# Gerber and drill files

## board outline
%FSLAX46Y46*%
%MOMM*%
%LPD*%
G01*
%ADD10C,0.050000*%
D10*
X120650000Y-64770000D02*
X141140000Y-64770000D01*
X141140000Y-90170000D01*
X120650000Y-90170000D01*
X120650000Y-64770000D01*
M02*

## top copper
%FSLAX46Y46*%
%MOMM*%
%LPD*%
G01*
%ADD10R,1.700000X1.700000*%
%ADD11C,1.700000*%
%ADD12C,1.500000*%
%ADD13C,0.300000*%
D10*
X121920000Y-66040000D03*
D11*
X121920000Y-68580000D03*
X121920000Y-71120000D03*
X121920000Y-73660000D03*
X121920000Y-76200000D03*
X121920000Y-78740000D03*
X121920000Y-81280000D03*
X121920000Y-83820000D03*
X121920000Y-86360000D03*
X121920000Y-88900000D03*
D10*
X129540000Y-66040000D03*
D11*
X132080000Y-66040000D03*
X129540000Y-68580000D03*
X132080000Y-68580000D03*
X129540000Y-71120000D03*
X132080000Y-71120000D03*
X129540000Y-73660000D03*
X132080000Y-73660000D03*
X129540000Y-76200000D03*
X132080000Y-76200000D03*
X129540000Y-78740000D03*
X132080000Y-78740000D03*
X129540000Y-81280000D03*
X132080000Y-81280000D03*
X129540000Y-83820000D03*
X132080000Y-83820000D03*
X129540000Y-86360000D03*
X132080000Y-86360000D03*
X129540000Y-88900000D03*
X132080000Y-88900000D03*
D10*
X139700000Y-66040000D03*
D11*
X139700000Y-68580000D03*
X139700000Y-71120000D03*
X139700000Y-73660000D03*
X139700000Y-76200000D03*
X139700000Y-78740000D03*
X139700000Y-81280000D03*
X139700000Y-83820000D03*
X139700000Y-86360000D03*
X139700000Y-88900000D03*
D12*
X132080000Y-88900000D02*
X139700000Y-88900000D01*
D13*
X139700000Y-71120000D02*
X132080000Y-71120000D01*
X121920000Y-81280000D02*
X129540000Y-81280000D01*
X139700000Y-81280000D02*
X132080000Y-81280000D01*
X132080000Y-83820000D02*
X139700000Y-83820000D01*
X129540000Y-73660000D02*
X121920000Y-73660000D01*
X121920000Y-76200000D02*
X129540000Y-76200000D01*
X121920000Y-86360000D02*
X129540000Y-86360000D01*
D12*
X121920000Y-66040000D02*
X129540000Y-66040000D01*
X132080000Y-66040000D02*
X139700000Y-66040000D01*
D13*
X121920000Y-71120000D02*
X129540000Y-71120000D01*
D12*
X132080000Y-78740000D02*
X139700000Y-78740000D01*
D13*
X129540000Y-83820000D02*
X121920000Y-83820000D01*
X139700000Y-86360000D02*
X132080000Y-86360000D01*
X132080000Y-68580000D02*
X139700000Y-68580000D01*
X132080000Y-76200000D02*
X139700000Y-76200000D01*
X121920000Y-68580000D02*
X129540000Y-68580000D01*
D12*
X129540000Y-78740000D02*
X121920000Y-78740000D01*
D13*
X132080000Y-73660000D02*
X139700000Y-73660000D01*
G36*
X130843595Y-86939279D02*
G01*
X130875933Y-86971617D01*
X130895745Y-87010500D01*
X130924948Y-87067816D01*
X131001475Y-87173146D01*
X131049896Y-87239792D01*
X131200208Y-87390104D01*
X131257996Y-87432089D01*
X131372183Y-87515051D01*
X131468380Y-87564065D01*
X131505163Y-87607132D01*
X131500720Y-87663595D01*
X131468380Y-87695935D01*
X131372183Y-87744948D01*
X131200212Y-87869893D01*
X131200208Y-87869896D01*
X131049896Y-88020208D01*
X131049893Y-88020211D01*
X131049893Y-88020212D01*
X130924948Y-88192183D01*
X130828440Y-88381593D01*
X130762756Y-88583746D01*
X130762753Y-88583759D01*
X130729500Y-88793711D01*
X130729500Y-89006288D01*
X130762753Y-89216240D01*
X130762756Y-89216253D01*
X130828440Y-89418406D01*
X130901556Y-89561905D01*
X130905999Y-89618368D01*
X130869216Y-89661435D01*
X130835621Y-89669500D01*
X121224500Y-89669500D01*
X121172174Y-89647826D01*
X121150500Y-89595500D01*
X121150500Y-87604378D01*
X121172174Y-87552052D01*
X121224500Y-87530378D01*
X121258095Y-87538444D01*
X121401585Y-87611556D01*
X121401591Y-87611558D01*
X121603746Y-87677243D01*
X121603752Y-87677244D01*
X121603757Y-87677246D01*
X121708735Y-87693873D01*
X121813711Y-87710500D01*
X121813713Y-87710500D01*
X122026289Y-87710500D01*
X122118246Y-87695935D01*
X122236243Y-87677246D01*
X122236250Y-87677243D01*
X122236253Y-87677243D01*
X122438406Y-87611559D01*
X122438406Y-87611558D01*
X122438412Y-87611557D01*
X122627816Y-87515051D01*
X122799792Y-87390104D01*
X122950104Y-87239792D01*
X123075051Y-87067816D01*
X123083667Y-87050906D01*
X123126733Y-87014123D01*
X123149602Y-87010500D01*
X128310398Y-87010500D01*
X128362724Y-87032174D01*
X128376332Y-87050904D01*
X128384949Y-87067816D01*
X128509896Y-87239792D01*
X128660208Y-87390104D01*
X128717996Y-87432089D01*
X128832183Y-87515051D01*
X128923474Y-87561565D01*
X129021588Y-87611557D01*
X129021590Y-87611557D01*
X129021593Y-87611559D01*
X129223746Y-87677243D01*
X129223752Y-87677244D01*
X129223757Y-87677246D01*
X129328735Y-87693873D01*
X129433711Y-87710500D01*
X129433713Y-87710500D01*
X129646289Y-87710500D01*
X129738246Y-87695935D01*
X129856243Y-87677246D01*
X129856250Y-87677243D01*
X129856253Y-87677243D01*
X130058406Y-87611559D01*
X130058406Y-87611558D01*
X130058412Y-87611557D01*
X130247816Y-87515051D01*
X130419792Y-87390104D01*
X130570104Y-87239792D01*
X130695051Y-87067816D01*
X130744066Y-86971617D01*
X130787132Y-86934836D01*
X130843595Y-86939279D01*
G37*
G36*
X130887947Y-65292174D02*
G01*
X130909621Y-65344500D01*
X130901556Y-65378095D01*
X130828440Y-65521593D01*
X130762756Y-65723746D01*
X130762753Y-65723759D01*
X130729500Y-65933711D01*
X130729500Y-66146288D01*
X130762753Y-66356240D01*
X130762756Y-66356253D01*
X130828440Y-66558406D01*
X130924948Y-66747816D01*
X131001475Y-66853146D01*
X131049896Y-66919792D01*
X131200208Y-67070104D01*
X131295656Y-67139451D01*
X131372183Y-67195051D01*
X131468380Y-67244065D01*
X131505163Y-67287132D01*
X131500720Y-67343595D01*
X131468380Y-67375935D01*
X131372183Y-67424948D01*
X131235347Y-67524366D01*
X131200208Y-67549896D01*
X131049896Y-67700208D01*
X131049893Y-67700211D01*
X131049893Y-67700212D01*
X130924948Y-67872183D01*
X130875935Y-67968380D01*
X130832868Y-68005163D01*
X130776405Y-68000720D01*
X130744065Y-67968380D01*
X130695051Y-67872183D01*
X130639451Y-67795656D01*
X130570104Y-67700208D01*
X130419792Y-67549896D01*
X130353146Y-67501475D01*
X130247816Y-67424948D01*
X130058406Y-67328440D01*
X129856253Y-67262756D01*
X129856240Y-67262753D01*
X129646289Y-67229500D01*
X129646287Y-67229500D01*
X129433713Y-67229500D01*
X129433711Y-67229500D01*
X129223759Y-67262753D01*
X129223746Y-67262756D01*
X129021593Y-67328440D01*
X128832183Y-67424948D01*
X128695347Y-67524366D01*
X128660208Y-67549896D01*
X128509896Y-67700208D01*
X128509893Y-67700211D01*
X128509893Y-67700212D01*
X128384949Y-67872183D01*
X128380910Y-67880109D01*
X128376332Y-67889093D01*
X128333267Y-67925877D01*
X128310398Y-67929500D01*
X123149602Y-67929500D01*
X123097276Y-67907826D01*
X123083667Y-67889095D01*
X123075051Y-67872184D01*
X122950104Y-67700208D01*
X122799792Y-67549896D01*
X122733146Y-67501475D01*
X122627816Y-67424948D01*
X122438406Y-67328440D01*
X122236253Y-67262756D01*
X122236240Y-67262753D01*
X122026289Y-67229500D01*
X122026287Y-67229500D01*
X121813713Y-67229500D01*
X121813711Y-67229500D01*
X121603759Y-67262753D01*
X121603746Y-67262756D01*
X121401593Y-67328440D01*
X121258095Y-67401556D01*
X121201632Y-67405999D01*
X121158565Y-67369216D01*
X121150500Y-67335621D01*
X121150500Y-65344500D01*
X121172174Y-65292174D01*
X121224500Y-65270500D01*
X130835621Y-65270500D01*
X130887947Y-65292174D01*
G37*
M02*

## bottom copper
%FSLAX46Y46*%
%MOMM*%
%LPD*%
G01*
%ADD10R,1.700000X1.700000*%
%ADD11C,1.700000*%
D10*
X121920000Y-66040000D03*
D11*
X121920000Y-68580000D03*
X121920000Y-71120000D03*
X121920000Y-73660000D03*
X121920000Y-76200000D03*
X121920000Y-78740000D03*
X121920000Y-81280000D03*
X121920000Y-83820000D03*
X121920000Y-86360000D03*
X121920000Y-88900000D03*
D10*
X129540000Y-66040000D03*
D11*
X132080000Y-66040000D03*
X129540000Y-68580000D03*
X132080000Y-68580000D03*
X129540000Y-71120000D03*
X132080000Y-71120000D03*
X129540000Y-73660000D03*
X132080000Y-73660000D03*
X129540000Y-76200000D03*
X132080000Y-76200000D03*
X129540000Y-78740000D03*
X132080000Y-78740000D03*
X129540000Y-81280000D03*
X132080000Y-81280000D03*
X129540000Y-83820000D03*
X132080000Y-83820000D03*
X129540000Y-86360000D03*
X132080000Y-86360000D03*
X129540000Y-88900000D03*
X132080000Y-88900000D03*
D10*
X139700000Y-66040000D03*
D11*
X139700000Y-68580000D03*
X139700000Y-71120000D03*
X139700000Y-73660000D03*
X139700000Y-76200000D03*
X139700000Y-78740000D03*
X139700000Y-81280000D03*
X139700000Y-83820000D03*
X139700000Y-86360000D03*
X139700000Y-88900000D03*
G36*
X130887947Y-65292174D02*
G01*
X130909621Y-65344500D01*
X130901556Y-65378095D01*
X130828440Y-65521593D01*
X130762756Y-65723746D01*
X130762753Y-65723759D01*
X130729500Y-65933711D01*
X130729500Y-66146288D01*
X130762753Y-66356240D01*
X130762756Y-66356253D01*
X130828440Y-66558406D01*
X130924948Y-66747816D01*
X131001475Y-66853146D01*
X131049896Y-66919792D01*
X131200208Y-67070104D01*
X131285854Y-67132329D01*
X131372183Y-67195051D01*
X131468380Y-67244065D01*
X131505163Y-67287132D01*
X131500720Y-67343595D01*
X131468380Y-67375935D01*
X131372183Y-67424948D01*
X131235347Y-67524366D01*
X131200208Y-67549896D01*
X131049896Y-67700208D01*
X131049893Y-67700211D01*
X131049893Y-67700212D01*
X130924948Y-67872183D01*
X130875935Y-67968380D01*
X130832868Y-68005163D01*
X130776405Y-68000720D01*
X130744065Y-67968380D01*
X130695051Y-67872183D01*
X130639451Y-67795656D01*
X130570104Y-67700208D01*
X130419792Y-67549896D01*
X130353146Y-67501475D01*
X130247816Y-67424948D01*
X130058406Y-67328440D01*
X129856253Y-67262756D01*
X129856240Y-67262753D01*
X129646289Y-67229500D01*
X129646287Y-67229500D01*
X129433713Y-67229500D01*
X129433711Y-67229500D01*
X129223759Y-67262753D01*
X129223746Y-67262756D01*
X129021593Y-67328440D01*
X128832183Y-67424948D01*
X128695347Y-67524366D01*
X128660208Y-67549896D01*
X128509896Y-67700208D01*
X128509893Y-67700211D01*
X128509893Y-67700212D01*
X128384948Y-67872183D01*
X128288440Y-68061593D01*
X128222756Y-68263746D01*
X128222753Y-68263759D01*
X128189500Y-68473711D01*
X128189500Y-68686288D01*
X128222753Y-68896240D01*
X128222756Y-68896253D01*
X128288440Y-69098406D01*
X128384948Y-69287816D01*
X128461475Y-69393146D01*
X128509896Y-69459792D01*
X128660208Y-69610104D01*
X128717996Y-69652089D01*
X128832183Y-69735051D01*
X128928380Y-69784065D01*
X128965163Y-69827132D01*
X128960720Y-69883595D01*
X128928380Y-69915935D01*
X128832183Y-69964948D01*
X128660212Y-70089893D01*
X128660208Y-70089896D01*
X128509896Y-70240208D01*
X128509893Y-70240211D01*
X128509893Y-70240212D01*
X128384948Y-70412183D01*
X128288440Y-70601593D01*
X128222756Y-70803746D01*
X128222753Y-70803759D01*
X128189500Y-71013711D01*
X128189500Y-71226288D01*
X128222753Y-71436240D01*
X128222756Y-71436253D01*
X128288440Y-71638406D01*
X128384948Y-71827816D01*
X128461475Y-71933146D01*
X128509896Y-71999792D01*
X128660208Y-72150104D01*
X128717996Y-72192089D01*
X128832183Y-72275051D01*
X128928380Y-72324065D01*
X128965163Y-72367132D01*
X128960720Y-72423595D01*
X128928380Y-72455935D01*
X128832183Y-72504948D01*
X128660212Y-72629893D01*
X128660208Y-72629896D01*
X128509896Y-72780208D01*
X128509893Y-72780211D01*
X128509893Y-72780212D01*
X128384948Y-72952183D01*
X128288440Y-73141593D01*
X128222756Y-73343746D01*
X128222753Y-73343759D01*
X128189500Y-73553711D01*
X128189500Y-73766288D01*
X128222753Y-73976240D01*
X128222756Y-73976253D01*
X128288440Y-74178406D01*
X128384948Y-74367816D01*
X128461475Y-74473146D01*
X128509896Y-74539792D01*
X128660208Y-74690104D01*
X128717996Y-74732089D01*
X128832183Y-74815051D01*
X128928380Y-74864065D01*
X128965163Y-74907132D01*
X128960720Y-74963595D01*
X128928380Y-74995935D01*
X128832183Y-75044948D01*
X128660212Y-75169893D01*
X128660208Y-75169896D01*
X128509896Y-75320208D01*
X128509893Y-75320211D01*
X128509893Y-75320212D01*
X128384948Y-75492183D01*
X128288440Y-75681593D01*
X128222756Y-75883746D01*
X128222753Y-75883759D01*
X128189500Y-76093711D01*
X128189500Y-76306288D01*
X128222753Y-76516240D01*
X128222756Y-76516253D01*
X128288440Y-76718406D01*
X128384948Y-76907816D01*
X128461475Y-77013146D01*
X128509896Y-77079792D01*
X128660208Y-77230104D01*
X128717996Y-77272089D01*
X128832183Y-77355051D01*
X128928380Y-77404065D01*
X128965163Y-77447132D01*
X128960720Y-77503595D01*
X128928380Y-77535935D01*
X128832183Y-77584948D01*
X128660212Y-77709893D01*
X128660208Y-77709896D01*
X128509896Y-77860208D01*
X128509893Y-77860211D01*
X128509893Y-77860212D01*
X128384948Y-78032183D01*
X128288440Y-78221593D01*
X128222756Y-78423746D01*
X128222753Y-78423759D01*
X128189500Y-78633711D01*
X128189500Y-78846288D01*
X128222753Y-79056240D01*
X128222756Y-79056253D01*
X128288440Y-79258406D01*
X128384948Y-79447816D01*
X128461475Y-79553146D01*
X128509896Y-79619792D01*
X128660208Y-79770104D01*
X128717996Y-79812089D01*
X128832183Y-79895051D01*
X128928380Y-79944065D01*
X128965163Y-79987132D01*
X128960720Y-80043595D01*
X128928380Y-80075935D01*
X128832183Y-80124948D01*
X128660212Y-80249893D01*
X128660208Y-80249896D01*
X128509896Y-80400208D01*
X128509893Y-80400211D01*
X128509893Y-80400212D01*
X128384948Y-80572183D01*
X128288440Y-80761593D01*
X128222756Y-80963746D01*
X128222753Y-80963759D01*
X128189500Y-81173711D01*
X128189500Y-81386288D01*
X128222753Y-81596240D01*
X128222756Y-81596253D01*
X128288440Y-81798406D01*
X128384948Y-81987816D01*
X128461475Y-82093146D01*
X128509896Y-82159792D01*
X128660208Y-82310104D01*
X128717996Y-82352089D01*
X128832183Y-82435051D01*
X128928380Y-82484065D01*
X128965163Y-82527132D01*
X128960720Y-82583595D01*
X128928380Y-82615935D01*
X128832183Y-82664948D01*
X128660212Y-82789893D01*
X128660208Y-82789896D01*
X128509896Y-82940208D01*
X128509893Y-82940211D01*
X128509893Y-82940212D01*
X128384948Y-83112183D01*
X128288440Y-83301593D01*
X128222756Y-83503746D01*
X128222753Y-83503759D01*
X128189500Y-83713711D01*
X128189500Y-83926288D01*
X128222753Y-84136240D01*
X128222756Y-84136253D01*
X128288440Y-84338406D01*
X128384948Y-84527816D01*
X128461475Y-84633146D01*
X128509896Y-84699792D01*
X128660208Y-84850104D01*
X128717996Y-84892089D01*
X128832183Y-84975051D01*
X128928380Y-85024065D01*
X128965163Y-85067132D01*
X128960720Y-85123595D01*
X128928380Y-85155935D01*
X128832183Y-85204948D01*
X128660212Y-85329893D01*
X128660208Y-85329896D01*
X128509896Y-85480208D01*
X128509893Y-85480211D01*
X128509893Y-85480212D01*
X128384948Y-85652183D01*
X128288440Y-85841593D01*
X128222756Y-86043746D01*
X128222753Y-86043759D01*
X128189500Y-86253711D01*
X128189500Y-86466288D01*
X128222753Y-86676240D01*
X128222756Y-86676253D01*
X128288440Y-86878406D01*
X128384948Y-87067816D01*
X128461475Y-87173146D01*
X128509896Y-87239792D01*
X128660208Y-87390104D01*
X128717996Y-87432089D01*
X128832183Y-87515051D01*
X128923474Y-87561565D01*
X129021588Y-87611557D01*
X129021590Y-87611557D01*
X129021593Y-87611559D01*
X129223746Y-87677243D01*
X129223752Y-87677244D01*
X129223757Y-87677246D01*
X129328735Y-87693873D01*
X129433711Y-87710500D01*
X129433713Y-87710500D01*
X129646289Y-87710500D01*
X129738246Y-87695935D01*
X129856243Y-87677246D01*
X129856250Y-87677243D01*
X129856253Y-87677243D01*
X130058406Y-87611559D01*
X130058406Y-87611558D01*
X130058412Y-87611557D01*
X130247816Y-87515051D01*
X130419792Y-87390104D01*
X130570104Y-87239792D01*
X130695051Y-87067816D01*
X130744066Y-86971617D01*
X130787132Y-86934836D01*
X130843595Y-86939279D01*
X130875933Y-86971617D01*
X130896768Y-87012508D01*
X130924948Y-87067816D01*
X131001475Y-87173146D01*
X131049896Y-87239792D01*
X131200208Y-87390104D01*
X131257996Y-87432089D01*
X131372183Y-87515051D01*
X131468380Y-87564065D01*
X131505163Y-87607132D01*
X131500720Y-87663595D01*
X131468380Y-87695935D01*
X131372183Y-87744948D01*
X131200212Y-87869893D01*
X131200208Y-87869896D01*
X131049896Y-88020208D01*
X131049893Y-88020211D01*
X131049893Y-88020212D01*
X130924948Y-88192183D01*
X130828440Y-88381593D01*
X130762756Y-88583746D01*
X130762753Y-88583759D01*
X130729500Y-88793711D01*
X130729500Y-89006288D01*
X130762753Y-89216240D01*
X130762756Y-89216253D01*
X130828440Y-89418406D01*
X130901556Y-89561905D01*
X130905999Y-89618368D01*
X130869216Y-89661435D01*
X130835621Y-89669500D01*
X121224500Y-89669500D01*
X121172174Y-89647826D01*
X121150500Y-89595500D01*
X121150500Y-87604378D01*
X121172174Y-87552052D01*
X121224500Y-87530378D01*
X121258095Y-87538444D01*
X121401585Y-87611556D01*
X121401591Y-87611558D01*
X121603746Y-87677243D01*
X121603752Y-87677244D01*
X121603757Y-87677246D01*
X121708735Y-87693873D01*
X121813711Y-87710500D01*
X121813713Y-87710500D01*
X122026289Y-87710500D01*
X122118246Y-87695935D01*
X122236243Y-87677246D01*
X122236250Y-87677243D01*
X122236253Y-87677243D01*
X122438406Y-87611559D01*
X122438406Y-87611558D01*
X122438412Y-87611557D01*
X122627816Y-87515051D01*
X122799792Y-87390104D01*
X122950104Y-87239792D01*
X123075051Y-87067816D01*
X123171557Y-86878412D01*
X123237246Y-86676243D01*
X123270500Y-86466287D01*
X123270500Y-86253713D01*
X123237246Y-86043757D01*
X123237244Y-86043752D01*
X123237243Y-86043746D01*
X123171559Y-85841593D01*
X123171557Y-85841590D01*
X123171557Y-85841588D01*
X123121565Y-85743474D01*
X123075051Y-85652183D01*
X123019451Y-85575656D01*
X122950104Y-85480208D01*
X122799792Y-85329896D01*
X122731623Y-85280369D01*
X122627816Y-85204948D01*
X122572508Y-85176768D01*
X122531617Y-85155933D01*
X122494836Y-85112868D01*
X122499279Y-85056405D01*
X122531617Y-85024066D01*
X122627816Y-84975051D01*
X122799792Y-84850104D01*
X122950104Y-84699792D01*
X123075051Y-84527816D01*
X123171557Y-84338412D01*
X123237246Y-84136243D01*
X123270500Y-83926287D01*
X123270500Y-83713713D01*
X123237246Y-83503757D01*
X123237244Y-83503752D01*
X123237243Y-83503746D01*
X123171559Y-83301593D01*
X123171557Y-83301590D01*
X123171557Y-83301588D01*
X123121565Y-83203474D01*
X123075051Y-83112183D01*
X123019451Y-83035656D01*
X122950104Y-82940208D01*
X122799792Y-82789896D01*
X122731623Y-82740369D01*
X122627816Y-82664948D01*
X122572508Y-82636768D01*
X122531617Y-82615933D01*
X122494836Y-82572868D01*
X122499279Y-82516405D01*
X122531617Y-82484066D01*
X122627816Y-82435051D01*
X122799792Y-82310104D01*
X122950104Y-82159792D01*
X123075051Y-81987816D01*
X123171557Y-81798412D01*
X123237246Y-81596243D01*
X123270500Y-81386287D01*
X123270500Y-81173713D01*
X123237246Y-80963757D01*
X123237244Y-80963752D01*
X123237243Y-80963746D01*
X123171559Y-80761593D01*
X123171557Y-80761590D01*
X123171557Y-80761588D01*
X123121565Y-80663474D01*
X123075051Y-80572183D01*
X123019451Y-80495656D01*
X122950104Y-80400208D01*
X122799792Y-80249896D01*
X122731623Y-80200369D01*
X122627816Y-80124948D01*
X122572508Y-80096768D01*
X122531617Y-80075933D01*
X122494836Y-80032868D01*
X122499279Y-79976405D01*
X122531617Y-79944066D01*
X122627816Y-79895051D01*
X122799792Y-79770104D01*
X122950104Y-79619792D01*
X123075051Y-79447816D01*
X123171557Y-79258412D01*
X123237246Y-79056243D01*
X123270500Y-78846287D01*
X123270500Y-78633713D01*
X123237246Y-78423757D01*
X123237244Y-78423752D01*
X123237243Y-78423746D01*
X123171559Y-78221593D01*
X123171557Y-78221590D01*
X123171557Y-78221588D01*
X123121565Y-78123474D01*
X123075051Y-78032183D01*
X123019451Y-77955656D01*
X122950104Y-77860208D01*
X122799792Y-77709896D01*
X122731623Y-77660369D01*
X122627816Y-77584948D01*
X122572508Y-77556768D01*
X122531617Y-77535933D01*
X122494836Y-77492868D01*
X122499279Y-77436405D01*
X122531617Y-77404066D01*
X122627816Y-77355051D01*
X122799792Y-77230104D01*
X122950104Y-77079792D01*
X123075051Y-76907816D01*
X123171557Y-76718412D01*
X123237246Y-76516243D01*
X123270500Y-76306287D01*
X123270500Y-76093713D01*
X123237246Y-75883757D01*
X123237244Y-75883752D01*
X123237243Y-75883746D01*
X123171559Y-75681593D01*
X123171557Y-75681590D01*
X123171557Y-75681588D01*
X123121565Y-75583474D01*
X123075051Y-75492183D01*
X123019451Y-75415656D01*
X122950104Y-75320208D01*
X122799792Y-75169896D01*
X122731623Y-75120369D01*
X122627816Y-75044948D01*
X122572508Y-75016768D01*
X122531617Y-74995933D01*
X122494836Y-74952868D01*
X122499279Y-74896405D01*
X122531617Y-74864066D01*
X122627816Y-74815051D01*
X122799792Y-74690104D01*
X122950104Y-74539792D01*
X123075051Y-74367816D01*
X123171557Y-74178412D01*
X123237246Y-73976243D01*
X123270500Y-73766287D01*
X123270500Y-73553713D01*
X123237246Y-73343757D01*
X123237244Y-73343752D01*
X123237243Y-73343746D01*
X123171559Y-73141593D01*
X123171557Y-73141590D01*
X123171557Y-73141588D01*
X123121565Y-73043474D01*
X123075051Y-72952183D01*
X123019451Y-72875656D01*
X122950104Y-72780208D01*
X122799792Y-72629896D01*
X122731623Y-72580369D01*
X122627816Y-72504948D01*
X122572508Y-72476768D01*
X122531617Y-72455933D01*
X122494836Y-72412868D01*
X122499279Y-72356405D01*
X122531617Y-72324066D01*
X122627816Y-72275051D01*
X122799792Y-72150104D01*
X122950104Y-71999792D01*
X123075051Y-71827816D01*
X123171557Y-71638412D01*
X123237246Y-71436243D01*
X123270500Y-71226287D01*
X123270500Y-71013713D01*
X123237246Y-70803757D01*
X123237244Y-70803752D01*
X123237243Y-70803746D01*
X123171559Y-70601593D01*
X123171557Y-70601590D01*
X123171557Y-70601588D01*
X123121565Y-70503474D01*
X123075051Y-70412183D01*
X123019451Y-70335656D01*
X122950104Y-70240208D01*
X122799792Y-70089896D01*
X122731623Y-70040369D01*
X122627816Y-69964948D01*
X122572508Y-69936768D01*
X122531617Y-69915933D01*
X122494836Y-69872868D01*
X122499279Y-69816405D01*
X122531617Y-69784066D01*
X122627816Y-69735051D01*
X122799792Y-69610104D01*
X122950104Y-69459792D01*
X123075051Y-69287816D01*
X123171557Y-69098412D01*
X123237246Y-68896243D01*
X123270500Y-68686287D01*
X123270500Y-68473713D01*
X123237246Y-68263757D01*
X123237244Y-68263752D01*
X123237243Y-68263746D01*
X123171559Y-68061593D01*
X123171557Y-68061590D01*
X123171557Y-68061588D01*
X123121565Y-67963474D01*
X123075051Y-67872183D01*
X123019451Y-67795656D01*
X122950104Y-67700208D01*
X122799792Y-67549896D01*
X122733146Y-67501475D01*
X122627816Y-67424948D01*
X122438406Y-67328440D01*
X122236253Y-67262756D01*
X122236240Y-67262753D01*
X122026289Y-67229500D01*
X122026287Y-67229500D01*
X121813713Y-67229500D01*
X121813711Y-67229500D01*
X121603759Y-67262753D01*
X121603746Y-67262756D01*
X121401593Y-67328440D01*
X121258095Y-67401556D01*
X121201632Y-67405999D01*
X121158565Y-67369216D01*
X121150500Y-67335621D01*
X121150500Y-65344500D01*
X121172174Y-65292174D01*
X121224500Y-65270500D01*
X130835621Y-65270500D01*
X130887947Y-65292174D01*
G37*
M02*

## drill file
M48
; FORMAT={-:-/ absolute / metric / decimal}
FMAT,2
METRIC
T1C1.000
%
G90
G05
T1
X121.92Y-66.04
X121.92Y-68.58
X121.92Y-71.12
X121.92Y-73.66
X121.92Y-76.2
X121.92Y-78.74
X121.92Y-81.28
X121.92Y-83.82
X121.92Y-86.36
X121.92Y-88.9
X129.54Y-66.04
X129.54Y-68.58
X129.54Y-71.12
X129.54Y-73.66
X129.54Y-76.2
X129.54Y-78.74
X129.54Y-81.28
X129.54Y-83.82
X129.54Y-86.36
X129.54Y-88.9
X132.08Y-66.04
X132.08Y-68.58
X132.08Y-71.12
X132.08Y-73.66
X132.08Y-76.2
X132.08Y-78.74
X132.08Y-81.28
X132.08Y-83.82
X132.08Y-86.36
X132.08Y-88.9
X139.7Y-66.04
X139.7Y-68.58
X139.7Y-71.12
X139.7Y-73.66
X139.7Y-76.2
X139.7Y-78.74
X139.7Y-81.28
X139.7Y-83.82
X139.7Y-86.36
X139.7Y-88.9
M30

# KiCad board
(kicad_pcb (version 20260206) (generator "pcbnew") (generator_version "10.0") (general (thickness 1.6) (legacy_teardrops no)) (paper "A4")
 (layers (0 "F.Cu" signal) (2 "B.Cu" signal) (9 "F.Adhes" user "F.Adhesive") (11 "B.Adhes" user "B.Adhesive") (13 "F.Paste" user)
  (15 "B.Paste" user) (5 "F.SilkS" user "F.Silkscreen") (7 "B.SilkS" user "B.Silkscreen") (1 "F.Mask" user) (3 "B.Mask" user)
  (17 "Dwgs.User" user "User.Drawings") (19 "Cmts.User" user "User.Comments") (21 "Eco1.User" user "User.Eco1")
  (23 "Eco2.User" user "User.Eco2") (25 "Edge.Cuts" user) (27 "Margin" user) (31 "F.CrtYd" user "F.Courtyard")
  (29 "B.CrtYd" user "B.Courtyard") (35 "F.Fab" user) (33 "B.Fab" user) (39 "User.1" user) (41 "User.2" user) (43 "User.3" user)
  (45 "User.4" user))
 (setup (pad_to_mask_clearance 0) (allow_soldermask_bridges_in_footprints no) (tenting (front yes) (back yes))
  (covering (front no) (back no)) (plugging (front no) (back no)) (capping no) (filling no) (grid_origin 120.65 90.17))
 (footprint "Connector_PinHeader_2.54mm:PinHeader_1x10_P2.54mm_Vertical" (layer "F.Cu") (at 121.92 66.04)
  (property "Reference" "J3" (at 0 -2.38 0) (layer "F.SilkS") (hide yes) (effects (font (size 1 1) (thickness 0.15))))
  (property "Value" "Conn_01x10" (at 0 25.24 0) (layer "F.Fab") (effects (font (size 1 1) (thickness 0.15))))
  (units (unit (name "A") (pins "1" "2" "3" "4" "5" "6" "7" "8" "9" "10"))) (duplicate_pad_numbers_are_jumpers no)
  (pad "1" thru_hole rect (at 0 0) (size 1.7 1.7) (drill 1) (layers "*.Cu" "*.Mask") (remove_unused_layers no) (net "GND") (zone_connect 2))
  (pad "2" thru_hole circle (at 0 2.54) (size 1.7 1.7) (drill 1) (layers "*.Cu" "*.Mask") (remove_unused_layers no) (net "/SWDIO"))
  (pad "3" thru_hole circle (at 0 5.08) (size 1.7 1.7) (drill 1) (layers "*.Cu" "*.Mask") (remove_unused_layers no) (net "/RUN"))
  (pad "4" thru_hole circle (at 0 7.62) (size 1.7 1.7) (drill 1) (layers "*.Cu" "*.Mask") (remove_unused_layers no) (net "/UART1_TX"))
  (pad "5" thru_hole circle (at 0 10.16) (size 1.7 1.7) (drill 1) (layers "*.Cu" "*.Mask") (remove_unused_layers no) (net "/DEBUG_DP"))
  (pad "6" thru_hole circle (at 0 12.7) (size 1.7 1.7) (drill 1) (layers "*.Cu" "*.Mask") (remove_unused_layers no) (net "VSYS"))
  (pad "7" thru_hole circle (at 0 15.24) (size 1.7 1.7) (drill 1) (layers "*.Cu" "*.Mask") (remove_unused_layers no) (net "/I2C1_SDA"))
  (pad "8" thru_hole circle (at 0 17.78) (size 1.7 1.7) (drill 1) (layers "*.Cu" "*.Mask") (remove_unused_layers no) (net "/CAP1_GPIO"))
  (pad "9" thru_hole circle (at 0 20.32) (size 1.7 1.7) (drill 1) (layers "*.Cu" "*.Mask") (remove_unused_layers no) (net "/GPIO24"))
  (pad "10" thru_hole circle (at 0 22.86) (size 1.7 1.7) (drill 1) (layers "*.Cu" "*.Mask") (remove_unused_layers no) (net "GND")
   (zone_connect 2)))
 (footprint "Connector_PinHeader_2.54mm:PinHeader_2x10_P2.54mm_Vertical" (layer "F.Cu") (at 129.54 66.04)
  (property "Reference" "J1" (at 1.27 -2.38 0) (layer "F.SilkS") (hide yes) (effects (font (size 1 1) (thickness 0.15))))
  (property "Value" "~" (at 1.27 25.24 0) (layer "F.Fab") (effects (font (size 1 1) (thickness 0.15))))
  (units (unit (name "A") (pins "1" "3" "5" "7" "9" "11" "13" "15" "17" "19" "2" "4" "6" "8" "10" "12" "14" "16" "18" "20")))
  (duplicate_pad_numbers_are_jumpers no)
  (pad "1" thru_hole rect (at 0 0) (size 1.7 1.7) (drill 1) (layers "*.Cu" "*.Mask") (remove_unused_layers no) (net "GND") (zone_connect 2))
  (pad "2" thru_hole circle (at 2.54 0) (size 1.7 1.7) (drill 1) (layers "*.Cu" "*.Mask") (remove_unused_layers no) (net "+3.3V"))
  (pad "3" thru_hole circle (at 0 2.54) (size 1.7 1.7) (drill 1) (layers "*.Cu" "*.Mask") (remove_unused_layers no) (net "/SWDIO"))
  (pad "4" thru_hole circle (at 2.54 2.54) (size 1.7 1.7) (drill 1) (layers "*.Cu" "*.Mask") (remove_unused_layers no) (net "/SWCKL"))
  (pad "5" thru_hole circle (at 0 5.08) (size 1.7 1.7) (drill 1) (layers "*.Cu" "*.Mask") (remove_unused_layers no) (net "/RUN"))
  (pad "6" thru_hole circle (at 2.54 5.08) (size 1.7 1.7) (drill 1) (layers "*.Cu" "*.Mask") (remove_unused_layers no) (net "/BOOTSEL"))
  (pad "7" thru_hole circle (at 0 7.62) (size 1.7 1.7) (drill 1) (layers "*.Cu" "*.Mask") (remove_unused_layers no) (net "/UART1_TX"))
  (pad "8" thru_hole circle (at 2.54 7.62) (size 1.7 1.7) (drill 1) (layers "*.Cu" "*.Mask") (remove_unused_layers no) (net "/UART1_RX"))
  (pad "9" thru_hole circle (at 0 10.16) (size 1.7 1.7) (drill 1) (layers "*.Cu" "*.Mask") (remove_unused_layers no) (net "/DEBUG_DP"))
  (pad "10" thru_hole circle (at 2.54 10.16) (size 1.7 1.7) (drill 1) (layers "*.Cu" "*.Mask") (remove_unused_layers no) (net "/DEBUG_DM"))
  (pad "11" thru_hole circle (at 0 12.7) (size 1.7 1.7) (drill 1) (layers "*.Cu" "*.Mask") (remove_unused_layers no) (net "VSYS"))
  (pad "12" thru_hole circle (at 2.54 12.7) (size 1.7 1.7) (drill 1) (layers "*.Cu" "*.Mask") (remove_unused_layers no) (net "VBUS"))
  (pad "13" thru_hole circle (at 0 15.24) (size 1.7 1.7) (drill 1) (layers "*.Cu" "*.Mask") (remove_unused_layers no) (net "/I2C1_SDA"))
  (pad "14" thru_hole circle (at 2.54 15.24) (size 1.7 1.7) (drill 1) (layers "*.Cu" "*.Mask") (remove_unused_layers no) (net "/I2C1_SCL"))
  (pad "15" thru_hole circle (at 0 17.78) (size 1.7 1.7) (drill 1) (layers "*.Cu" "*.Mask") (remove_unused_layers no) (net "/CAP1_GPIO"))
  (pad "16" thru_hole circle (at 2.54 17.78) (size 1.7 1.7) (drill 1) (layers "*.Cu" "*.Mask") (remove_unused_layers no) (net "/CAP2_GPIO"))
  (pad "17" thru_hole circle (at 0 20.32) (size 1.7 1.7) (drill 1) (layers "*.Cu" "*.Mask") (remove_unused_layers no) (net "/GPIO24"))
  (pad "18" thru_hole circle (at 2.54 20.32) (size 1.7 1.7) (drill 1) (layers "*.Cu" "*.Mask") (remove_unused_layers no) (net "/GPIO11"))
  (pad "19" thru_hole circle (at 0 22.86) (size 1.7 1.7) (drill 1) (layers "*.Cu" "*.Mask") (remove_unused_layers no) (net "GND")
   (zone_connect 2))
  (pad "20" thru_hole circle (at 2.54 22.86) (size 1.7 1.7) (drill 1) (layers "*.Cu" "*.Mask") (remove_unused_layers no) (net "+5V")))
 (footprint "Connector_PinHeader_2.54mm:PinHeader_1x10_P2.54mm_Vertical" (layer "F.Cu") (at 139.7 66.04)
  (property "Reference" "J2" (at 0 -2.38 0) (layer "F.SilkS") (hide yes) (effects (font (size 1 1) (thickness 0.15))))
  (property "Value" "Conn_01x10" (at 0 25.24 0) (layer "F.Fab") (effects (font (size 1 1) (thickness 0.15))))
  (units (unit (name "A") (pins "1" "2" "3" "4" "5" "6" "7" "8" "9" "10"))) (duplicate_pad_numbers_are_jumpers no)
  (pad "1" thru_hole rect (at 0 0) (size 1.7 1.7) (drill 1) (layers "*.Cu" "*.Mask") (remove_unused_layers no) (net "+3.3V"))
  (pad "2" thru_hole circle (at 0 2.54) (size 1.7 1.7) (drill 1) (layers "*.Cu" "*.Mask") (remove_unused_layers no) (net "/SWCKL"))
  (pad "3" thru_hole circle (at 0 5.08) (size 1.7 1.7) (drill 1) (layers "*.Cu" "*.Mask") (remove_unused_layers no) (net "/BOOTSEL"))
  (pad "4" thru_hole circle (at 0 7.62) (size 1.7 1.7) (drill 1) (layers "*.Cu" "*.Mask") (remove_unused_layers no) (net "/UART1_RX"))
  (pad "5" thru_hole circle (at 0 10.16) (size 1.7 1.7) (drill 1) (layers "*.Cu" "*.Mask") (remove_unused_layers no) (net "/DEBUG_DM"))
  (pad "6" thru_hole circle (at 0 12.7) (size 1.7 1.7) (drill 1) (layers "*.Cu" "*.Mask") (remove_unused_layers no) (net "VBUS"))
  (pad "7" thru_hole circle (at 0 15.24) (size 1.7 1.7) (drill 1) (layers "*.Cu" "*.Mask") (remove_unused_layers no) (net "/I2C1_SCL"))
  (pad "8" thru_hole circle (at 0 17.78) (size 1.7 1.7) (drill 1) (layers "*.Cu" "*.Mask") (remove_unused_layers no) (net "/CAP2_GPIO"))
  (pad "9" thru_hole circle (at 0 20.32) (size 1.7 1.7) (drill 1) (layers "*.Cu" "*.Mask") (remove_unused_layers no) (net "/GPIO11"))
  (pad "10" thru_hole circle (at 0 22.86) (size 1.7 1.7) (drill 1) (layers "*.Cu" "*.Mask") (remove_unused_layers no) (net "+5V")))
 (gr_rect (start 120.65 64.77) (end 141.14 90.17) (stroke (width 0.05) (type default)) (fill no) (layer "Edge.Cuts"))
 (segment (start 132.08 88.9) (end 139.7 88.9) (width 1.5) (layer "F.Cu") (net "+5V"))
 (segment (start 139.7 71.12) (end 132.08 71.12) (width 0.3) (layer "F.Cu") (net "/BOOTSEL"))
 (segment (start 121.92 81.28) (end 129.54 81.28) (width 0.3) (layer "F.Cu") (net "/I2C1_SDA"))
 (segment (start 139.7 81.28) (end 132.08 81.28) (width 0.3) (layer "F.Cu") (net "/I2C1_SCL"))
 (segment (start 132.08 83.82) (end 139.7 83.82) (width 0.3) (layer "F.Cu") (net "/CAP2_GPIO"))
 (segment (start 129.54 73.66) (end 121.92 73.66) (width 0.3) (layer "F.Cu") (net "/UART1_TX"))
 (segment (start 121.92 76.2) (end 129.54 76.2) (width 0.3) (layer "F.Cu") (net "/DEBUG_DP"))
 (segment (start 121.92 86.36) (end 129.54 86.36) (width 0.3) (layer "F.Cu") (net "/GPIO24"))
 (segment (start 121.92 66.04) (end 129.54 66.04) (width 1.5) (layer "F.Cu") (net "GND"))
 (segment (start 132.08 66.04) (end 139.7 66.04) (width 1.5) (layer "F.Cu") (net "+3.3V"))
 (segment (start 121.92 71.12) (end 129.54 71.12) (width 0.3) (layer "F.Cu") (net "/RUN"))
 (segment (start 132.08 78.74) (end 139.7 78.74) (width 1.5) (layer "F.Cu") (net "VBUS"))
 (segment (start 129.54 83.82) (end 121.92 83.82) (width 0.3) (layer "F.Cu") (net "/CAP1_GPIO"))
 (segment (start 139.7 86.36) (end 132.08 86.36) (width 0.3) (layer "F.Cu") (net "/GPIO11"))
 (segment (start 132.08 68.58) (end 139.7 68.58) (width 0.3) (layer "F.Cu") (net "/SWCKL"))
 (segment (start 132.08 76.2) (end 139.7 76.2) (width 0.3) (layer "F.Cu") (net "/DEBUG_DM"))
 (segment (start 121.92 68.58) (end 129.54 68.58) (width 0.3) (layer "F.Cu") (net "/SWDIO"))
 (segment (start 129.54 78.74) (end 121.92 78.74) (width 1.5) (layer "F.Cu") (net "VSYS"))
 (segment (start 132.08 73.66) (end 139.7 73.66) (width 0.3) (layer "F.Cu") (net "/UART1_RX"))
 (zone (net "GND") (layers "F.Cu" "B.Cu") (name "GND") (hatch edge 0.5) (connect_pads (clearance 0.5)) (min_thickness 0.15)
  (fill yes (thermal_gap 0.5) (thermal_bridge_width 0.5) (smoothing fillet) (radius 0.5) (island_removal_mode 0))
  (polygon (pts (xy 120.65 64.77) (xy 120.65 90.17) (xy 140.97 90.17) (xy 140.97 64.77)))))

